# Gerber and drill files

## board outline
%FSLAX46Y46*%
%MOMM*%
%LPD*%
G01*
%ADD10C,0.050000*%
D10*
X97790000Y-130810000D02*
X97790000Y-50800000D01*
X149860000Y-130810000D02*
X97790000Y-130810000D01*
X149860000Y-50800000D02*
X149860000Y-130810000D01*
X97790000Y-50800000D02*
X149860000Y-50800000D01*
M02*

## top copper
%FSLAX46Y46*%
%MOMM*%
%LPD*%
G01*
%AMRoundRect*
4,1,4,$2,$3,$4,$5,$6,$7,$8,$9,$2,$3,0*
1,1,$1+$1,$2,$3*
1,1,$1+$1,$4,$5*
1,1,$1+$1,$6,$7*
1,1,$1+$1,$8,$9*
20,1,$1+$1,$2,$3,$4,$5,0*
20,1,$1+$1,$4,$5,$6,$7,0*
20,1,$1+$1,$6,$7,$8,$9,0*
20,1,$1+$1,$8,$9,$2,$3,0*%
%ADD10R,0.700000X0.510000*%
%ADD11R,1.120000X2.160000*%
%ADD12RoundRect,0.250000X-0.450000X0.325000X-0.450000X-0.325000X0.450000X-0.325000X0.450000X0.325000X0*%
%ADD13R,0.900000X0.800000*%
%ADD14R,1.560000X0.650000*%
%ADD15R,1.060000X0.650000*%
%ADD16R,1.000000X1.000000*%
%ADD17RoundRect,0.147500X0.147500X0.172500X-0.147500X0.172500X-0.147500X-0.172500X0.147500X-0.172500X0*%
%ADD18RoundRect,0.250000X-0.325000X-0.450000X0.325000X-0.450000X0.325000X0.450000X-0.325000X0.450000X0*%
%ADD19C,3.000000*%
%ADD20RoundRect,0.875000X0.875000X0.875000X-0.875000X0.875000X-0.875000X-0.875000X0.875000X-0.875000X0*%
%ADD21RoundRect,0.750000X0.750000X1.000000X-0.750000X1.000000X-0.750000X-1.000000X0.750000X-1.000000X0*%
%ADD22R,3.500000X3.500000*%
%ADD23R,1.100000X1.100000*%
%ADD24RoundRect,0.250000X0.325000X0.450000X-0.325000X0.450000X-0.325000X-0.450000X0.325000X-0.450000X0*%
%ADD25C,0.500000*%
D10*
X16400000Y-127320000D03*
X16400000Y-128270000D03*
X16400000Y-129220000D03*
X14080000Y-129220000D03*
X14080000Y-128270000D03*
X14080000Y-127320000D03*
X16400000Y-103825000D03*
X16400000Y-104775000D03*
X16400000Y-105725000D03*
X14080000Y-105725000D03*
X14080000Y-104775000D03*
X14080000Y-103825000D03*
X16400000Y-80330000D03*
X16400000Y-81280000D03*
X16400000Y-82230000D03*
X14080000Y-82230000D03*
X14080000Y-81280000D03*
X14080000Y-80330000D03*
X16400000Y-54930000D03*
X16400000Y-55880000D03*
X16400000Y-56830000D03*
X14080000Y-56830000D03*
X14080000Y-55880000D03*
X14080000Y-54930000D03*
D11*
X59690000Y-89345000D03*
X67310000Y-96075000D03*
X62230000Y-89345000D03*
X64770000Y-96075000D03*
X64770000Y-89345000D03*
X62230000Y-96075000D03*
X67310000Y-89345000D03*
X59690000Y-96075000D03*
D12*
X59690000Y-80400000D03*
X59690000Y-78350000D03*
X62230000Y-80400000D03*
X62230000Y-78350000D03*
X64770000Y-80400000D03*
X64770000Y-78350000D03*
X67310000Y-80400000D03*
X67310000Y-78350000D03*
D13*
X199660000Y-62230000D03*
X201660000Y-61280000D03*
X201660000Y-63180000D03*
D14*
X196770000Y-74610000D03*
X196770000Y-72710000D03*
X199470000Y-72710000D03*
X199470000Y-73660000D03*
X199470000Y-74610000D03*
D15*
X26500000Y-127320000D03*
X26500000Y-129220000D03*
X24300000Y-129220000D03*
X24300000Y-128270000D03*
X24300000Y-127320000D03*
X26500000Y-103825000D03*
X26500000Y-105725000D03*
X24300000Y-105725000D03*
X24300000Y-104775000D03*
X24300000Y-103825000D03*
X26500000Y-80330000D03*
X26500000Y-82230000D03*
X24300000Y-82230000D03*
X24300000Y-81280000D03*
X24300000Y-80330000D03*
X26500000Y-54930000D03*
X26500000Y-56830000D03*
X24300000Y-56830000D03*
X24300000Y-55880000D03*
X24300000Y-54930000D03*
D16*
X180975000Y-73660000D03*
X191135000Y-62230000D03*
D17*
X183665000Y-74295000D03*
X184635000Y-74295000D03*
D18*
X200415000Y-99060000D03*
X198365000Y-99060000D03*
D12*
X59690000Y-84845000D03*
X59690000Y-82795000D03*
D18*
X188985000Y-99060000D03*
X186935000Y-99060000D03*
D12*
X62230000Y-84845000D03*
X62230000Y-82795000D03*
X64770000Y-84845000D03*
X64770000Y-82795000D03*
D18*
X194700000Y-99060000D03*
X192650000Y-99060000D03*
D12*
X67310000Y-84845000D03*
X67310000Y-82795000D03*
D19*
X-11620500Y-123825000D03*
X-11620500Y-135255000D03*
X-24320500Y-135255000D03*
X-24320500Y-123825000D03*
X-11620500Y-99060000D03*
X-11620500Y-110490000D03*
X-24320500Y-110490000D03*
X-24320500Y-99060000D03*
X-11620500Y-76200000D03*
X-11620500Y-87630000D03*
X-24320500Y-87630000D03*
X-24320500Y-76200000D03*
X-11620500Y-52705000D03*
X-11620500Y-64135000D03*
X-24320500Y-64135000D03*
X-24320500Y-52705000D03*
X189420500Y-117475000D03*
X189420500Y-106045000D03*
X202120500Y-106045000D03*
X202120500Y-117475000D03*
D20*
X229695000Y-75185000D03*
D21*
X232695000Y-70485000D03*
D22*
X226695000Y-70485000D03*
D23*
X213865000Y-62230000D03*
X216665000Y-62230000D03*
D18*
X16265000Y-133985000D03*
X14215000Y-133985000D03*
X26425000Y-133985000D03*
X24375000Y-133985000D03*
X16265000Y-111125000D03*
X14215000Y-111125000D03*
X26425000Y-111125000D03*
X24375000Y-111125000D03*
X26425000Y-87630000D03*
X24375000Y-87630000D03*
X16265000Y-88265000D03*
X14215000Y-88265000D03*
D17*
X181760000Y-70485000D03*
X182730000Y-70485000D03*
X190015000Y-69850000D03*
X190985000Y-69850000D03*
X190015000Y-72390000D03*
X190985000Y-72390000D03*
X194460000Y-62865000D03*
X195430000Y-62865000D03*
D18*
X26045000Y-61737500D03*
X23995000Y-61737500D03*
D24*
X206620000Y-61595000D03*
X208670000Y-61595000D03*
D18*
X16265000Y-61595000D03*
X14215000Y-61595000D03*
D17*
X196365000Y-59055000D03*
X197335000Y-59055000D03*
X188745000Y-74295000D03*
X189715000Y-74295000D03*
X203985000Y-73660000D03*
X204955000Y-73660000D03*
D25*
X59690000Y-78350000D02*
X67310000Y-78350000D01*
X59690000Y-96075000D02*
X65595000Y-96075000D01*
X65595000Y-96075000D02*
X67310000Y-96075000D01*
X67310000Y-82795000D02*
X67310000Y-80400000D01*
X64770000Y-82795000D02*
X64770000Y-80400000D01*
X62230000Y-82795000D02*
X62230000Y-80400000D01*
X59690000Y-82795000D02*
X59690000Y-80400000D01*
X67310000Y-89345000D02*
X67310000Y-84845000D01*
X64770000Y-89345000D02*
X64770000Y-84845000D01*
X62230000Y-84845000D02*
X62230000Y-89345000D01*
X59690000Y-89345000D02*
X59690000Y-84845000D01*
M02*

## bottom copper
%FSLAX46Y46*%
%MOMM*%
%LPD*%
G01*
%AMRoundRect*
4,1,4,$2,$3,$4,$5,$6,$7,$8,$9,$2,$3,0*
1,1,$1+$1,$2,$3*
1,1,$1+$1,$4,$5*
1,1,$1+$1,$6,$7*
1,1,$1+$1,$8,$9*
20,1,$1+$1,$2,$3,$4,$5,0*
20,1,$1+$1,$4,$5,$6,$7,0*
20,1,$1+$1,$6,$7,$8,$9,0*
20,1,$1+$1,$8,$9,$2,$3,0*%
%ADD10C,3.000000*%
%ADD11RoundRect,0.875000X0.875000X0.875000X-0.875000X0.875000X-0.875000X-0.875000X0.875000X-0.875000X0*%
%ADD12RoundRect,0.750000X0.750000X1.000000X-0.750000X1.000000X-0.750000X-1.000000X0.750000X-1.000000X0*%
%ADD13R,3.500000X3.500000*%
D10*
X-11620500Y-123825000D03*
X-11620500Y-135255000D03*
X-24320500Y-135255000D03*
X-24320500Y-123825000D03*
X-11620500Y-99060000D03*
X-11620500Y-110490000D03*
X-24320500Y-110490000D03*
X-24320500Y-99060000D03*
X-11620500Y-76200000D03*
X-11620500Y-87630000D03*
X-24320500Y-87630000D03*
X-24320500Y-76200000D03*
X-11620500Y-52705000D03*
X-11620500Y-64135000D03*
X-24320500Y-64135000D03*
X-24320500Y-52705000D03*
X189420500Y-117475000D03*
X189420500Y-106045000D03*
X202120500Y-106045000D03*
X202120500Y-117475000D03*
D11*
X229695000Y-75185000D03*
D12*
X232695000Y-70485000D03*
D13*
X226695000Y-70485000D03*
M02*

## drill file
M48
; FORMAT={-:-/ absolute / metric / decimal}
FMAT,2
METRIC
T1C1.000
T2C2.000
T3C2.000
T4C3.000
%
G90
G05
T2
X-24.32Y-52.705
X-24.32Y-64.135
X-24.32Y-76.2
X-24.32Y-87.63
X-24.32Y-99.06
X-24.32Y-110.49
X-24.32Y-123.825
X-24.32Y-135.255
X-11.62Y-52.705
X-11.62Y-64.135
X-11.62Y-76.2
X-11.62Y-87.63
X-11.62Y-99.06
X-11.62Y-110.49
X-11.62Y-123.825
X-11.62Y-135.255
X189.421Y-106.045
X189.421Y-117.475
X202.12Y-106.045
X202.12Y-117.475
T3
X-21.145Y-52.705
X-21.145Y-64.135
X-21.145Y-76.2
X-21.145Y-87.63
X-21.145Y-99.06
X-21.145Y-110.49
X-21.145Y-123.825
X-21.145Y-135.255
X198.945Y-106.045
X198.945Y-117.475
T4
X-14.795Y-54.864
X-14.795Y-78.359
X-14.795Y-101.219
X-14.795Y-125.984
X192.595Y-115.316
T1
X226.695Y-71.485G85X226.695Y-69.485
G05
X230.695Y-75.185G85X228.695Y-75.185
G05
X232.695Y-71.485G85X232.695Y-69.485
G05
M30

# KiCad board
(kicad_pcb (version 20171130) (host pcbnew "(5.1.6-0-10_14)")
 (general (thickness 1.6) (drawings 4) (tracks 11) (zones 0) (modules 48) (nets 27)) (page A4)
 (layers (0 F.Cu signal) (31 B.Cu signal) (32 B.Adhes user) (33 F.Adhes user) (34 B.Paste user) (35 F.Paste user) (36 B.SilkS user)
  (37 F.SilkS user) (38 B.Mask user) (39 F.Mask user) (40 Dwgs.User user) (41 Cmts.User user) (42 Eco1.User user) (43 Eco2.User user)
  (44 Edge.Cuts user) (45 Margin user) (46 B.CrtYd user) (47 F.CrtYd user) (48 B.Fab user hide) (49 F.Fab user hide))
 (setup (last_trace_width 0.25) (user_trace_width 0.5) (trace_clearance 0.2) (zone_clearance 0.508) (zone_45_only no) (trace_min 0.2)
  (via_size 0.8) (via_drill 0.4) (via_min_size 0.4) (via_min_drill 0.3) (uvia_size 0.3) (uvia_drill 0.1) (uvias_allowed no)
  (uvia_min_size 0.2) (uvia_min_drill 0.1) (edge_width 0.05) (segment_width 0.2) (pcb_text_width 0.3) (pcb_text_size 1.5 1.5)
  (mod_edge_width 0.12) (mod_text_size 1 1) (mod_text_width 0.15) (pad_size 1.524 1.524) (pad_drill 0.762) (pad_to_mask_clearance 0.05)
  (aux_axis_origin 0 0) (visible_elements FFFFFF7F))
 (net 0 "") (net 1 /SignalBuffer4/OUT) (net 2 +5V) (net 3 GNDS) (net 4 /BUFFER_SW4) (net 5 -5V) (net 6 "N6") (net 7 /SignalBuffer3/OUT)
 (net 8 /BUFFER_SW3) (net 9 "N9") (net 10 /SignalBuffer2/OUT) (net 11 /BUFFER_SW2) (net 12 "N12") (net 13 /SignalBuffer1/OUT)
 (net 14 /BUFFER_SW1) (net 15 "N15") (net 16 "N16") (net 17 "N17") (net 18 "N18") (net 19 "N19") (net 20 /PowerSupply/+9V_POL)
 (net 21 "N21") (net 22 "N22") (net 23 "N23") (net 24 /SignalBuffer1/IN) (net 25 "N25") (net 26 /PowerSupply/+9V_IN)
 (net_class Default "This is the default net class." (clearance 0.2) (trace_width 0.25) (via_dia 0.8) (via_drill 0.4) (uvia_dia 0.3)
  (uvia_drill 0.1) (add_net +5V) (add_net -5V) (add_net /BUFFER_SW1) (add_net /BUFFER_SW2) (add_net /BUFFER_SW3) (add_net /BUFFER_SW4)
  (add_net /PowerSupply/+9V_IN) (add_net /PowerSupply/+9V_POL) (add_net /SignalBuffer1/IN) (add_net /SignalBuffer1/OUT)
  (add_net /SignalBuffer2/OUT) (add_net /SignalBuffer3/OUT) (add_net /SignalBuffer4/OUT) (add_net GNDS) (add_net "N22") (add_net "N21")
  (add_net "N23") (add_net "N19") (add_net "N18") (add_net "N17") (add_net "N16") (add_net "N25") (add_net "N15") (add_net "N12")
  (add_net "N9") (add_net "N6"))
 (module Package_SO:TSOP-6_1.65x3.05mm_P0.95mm (layer F.Cu) (at 15.24 128.27)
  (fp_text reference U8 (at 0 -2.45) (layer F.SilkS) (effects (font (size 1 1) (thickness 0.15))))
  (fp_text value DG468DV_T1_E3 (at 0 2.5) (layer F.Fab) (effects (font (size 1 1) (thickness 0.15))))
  (pad 6 smd rect (at 1.16 -0.95) (size 0.7 0.51) (layers F.Cu F.Paste F.Mask) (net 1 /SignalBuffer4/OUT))
  (pad 5 smd rect (at 1.16 0) (size 0.7 0.51) (layers F.Cu F.Paste F.Mask) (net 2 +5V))
  (pad 4 smd rect (at 1.16 0.95) (size 0.7 0.51) (layers F.Cu F.Paste F.Mask) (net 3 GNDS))
  (pad 3 smd rect (at -1.16 0.95) (size 0.7 0.51) (layers F.Cu F.Paste F.Mask) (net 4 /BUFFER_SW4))
  (pad 2 smd rect (at -1.16 0) (size 0.7 0.51) (layers F.Cu F.Paste F.Mask) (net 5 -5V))
  (pad 1 smd rect (at -1.16 -0.95) (size 0.7 0.51) (layers F.Cu F.Paste F.Mask) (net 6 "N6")))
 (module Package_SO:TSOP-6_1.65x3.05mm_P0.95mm (layer F.Cu) (at 15.24 104.775)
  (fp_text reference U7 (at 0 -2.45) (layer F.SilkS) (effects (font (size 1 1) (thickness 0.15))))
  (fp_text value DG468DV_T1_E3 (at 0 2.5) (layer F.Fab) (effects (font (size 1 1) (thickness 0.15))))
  (pad 6 smd rect (at 1.16 -0.95) (size 0.7 0.51) (layers F.Cu F.Paste F.Mask) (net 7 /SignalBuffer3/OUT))
  (pad 5 smd rect (at 1.16 0) (size 0.7 0.51) (layers F.Cu F.Paste F.Mask) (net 2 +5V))
  (pad 4 smd rect (at 1.16 0.95) (size 0.7 0.51) (layers F.Cu F.Paste F.Mask) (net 3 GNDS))
  (pad 3 smd rect (at -1.16 0.95) (size 0.7 0.51) (layers F.Cu F.Paste F.Mask) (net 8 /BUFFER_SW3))
  (pad 2 smd rect (at -1.16 0) (size 0.7 0.51) (layers F.Cu F.Paste F.Mask) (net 5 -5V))
  (pad 1 smd rect (at -1.16 -0.95) (size 0.7 0.51) (layers F.Cu F.Paste F.Mask) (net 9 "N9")))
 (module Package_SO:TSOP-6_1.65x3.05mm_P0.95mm (layer F.Cu) (at 15.24 81.28)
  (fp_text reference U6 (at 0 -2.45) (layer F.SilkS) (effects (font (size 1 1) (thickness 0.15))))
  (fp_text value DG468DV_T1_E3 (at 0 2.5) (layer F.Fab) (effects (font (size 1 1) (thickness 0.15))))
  (pad 6 smd rect (at 1.16 -0.95) (size 0.7 0.51) (layers F.Cu F.Paste F.Mask) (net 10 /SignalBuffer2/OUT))
  (pad 5 smd rect (at 1.16 0) (size 0.7 0.51) (layers F.Cu F.Paste F.Mask) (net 2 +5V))
  (pad 4 smd rect (at 1.16 0.95) (size 0.7 0.51) (layers F.Cu F.Paste F.Mask) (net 3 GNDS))
  (pad 3 smd rect (at -1.16 0.95) (size 0.7 0.51) (layers F.Cu F.Paste F.Mask) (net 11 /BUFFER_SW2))
  (pad 2 smd rect (at -1.16 0) (size 0.7 0.51) (layers F.Cu F.Paste F.Mask) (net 5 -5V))
  (pad 1 smd rect (at -1.16 -0.95) (size 0.7 0.51) (layers F.Cu F.Paste F.Mask) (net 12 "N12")))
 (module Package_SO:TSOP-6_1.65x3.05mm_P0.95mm (layer F.Cu) (at 15.24 55.88)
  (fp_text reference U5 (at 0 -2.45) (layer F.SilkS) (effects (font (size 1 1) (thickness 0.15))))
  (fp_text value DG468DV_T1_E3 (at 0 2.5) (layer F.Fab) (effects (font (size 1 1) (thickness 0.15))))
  (pad 6 smd rect (at 1.16 -0.95) (size 0.7 0.51) (layers F.Cu F.Paste F.Mask) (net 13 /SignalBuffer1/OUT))
  (pad 5 smd rect (at 1.16 0) (size 0.7 0.51) (layers F.Cu F.Paste F.Mask) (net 2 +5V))
  (pad 4 smd rect (at 1.16 0.95) (size 0.7 0.51) (layers F.Cu F.Paste F.Mask) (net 3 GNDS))
  (pad 3 smd rect (at -1.16 0.95) (size 0.7 0.51) (layers F.Cu F.Paste F.Mask) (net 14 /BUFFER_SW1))
  (pad 2 smd rect (at -1.16 0) (size 0.7 0.51) (layers F.Cu F.Paste F.Mask) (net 5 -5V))
  (pad 1 smd rect (at -1.16 -0.95) (size 0.7 0.51) (layers F.Cu F.Paste F.Mask) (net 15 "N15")))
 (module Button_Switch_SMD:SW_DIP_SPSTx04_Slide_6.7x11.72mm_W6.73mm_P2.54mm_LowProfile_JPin (layer F.Cu) (at 63.5 92.71 90)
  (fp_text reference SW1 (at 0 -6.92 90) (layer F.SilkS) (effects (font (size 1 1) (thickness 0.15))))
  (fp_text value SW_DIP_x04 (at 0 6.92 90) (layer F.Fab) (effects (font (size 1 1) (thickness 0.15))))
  (pad 8 smd rect (at 3.365 -3.81 90) (size 2.16 1.12) (layers F.Cu F.Paste F.Mask) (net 14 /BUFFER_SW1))
  (pad 4 smd rect (at -3.365 3.81 90) (size 2.16 1.12) (layers F.Cu F.Paste F.Mask) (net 2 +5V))
  (pad 7 smd rect (at 3.365 -1.27 90) (size 2.16 1.12) (layers F.Cu F.Paste F.Mask) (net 11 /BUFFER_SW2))
  (pad 3 smd rect (at -3.365 1.27 90) (size 2.16 1.12) (layers F.Cu F.Paste F.Mask) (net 2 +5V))
  (pad 6 smd rect (at 3.365 1.27 90) (size 2.16 1.12) (layers F.Cu F.Paste F.Mask) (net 8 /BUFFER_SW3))
  (pad 2 smd rect (at -3.365 -1.27 90) (size 2.16 1.12) (layers F.Cu F.Paste F.Mask) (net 2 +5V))
  (pad 5 smd rect (at 3.365 3.81 90) (size 2.16 1.12) (layers F.Cu F.Paste F.Mask) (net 4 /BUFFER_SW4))
  (pad 1 smd rect (at -3.365 -3.81 90) (size 2.16 1.12) (layers F.Cu F.Paste F.Mask) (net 2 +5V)))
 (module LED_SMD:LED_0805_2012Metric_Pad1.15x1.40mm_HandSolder (layer F.Cu) (at 59.69 79.375 270)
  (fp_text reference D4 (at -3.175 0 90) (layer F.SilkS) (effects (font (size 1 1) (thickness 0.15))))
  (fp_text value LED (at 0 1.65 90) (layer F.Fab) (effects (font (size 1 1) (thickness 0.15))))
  (pad 2 smd roundrect (at 1.025 0 270) (size 1.15 1.4) (layers F.Cu F.Paste F.Mask) (roundrect_rratio 0.217391) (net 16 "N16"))
  (pad 1 smd roundrect (at -1.025 0 270) (size 1.15 1.4) (layers F.Cu F.Paste F.Mask) (roundrect_rratio 0.217391) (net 3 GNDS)))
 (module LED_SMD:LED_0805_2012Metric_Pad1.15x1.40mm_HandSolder (layer F.Cu) (at 62.23 79.375 270)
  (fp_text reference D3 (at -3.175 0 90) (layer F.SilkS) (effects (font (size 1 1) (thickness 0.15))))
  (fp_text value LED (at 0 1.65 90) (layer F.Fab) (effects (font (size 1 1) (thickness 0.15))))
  (pad 2 smd roundrect (at 1.025 0 270) (size 1.15 1.4) (layers F.Cu F.Paste F.Mask) (roundrect_rratio 0.217391) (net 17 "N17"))
  (pad 1 smd roundrect (at -1.025 0 270) (size 1.15 1.4) (layers F.Cu F.Paste F.Mask) (roundrect_rratio 0.217391) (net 3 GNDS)))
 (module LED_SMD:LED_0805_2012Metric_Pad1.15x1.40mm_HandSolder (layer F.Cu) (at 64.77 79.375 270)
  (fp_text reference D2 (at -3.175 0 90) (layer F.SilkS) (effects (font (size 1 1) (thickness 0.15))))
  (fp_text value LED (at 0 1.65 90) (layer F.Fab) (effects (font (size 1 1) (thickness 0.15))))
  (pad 2 smd roundrect (at 1.025 0 270) (size 1.15 1.4) (layers F.Cu F.Paste F.Mask) (roundrect_rratio 0.217391) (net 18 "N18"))
  (pad 1 smd roundrect (at -1.025 0 270) (size 1.15 1.4) (layers F.Cu F.Paste F.Mask) (roundrect_rratio 0.217391) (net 3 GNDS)))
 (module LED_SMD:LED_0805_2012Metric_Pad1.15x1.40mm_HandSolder (layer F.Cu) (at 67.31 79.375 270)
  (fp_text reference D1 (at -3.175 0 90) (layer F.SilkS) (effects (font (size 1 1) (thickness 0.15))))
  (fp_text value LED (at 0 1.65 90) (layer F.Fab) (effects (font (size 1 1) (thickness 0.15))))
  (pad 2 smd roundrect (at 1.025 0 270) (size 1.15 1.4) (layers F.Cu F.Paste F.Mask) (roundrect_rratio 0.217391) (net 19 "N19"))
  (pad 1 smd roundrect (at -1.025 0 270) (size 1.15 1.4) (layers F.Cu F.Paste F.Mask) (roundrect_rratio 0.217391) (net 3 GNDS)))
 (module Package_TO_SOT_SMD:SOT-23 (layer F.Cu) (at 200.66 62.23 180)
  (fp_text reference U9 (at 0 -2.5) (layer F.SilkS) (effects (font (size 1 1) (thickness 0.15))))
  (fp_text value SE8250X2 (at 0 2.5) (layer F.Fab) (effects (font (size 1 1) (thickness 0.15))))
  (pad 3 smd rect (at 1 0 180) (size 0.9 0.8) (layers F.Cu F.Paste F.Mask) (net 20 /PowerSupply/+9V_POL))
  (pad 2 smd rect (at -1 0.95 180) (size 0.9 0.8) (layers F.Cu F.Paste F.Mask) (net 2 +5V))
  (pad 1 smd rect (at -1 -0.95 180) (size 0.9 0.8) (layers F.Cu F.Paste F.Mask) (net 3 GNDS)))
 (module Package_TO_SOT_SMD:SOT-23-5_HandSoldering (layer F.Cu) (at 198.12 73.66 180)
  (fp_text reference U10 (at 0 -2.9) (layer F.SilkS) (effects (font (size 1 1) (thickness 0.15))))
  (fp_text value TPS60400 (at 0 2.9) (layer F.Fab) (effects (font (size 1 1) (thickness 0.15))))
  (pad 5 smd rect (at 1.35 -0.95 180) (size 1.56 0.65) (layers F.Cu F.Paste F.Mask) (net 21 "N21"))
  (pad 4 smd rect (at 1.35 0.95 180) (size 1.56 0.65) (layers F.Cu F.Paste F.Mask) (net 3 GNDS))
  (pad 3 smd rect (at -1.35 0.95 180) (size 1.56 0.65) (layers F.Cu F.Paste F.Mask) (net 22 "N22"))
  (pad 2 smd rect (at -1.35 0 180) (size 1.56 0.65) (layers F.Cu F.Paste F.Mask) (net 2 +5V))
  (pad 1 smd rect (at -1.35 -0.95 180) (size 1.56 0.65) (layers F.Cu F.Paste F.Mask) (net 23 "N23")))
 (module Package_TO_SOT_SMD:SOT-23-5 (layer F.Cu) (at 25.4 128.27)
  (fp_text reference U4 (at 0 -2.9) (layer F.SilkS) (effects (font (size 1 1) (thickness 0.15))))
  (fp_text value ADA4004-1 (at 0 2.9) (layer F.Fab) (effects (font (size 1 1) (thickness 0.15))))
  (pad 5 smd rect (at 1.1 -0.95) (size 1.06 0.65) (layers F.Cu F.Paste F.Mask) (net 2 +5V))
  (pad 4 smd rect (at 1.1 0.95) (size 1.06 0.65) (layers F.Cu F.Paste F.Mask) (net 6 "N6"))
  (pad 3 smd rect (at -1.1 0.95) (size 1.06 0.65) (layers F.Cu F.Paste F.Mask) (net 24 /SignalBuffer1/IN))
  (pad 2 smd rect (at -1.1 0) (size 1.06 0.65) (layers F.Cu F.Paste F.Mask) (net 5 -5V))
  (pad 1 smd rect (at -1.1 -0.95) (size 1.06 0.65) (layers F.Cu F.Paste F.Mask) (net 6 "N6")))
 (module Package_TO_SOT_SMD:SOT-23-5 (layer F.Cu) (at 25.4 104.775)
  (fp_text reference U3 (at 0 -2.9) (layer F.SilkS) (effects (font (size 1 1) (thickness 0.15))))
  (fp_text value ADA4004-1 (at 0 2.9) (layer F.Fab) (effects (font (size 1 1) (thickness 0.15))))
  (pad 5 smd rect (at 1.1 -0.95) (size 1.06 0.65) (layers F.Cu F.Paste F.Mask) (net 2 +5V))
  (pad 4 smd rect (at 1.1 0.95) (size 1.06 0.65) (layers F.Cu F.Paste F.Mask) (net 9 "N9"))
  (pad 3 smd rect (at -1.1 0.95) (size 1.06 0.65) (layers F.Cu F.Paste F.Mask) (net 24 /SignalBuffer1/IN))
  (pad 2 smd rect (at -1.1 0) (size 1.06 0.65) (layers F.Cu F.Paste F.Mask) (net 5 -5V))
  (pad 1 smd rect (at -1.1 -0.95) (size 1.06 0.65) (layers F.Cu F.Paste F.Mask) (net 9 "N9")))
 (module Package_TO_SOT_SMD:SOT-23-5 (layer F.Cu) (at 25.4 81.28)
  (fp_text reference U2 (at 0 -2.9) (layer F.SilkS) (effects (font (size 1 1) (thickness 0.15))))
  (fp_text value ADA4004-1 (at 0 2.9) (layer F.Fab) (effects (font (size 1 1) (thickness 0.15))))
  (pad 5 smd rect (at 1.1 -0.95) (size 1.06 0.65) (layers F.Cu F.Paste F.Mask) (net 2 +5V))
  (pad 4 smd rect (at 1.1 0.95) (size 1.06 0.65) (layers F.Cu F.Paste F.Mask) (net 12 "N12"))
  (pad 3 smd rect (at -1.1 0.95) (size 1.06 0.65) (layers F.Cu F.Paste F.Mask) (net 24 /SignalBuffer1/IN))
  (pad 2 smd rect (at -1.1 0) (size 1.06 0.65) (layers F.Cu F.Paste F.Mask) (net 5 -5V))
  (pad 1 smd rect (at -1.1 -0.95) (size 1.06 0.65) (layers F.Cu F.Paste F.Mask) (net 12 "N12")))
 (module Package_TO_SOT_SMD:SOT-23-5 (layer F.Cu) (at 25.4 55.88)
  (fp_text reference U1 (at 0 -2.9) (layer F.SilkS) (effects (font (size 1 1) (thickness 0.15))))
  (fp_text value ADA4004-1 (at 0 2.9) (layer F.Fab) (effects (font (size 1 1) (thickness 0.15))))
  (pad 5 smd rect (at 1.1 -0.95) (size 1.06 0.65) (layers F.Cu F.Paste F.Mask) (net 2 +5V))
  (pad 4 smd rect (at 1.1 0.95) (size 1.06 0.65) (layers F.Cu F.Paste F.Mask) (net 15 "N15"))
  (pad 3 smd rect (at -1.1 0.95) (size 1.06 0.65) (layers F.Cu F.Paste F.Mask) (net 24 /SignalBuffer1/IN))
  (pad 2 smd rect (at -1.1 0) (size 1.06 0.65) (layers F.Cu F.Paste F.Mask) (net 5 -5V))
  (pad 1 smd rect (at -1.1 -0.95) (size 1.06 0.65) (layers F.Cu F.Paste F.Mask) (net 15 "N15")))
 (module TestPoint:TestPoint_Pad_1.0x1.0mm (layer F.Cu) (at 180.975 73.66 180)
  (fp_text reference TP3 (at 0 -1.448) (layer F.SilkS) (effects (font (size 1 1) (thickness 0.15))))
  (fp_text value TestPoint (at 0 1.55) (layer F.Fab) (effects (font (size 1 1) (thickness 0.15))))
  (pad 1 smd rect (at 0 0 180) (size 1 1) (layers F.Cu F.Mask) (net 5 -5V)))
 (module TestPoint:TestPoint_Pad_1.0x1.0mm (layer F.Cu) (at 191.135 62.23 180)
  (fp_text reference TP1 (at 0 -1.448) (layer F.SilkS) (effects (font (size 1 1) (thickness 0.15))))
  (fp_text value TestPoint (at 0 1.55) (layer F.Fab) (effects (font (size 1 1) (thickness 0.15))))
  (pad 1 smd rect (at 0 0 180) (size 1 1) (layers F.Cu F.Mask) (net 2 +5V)))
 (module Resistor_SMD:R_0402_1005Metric (layer F.Cu) (at 184.15 74.295 180)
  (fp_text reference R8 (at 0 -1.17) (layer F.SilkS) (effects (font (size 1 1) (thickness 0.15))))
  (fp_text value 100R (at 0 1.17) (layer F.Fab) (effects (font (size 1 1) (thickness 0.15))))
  (pad 2 smd roundrect (at 0.485 0 180) (size 0.59 0.64) (layers F.Cu F.Paste F.Mask) (roundrect_rratio 0.25) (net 5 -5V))
  (pad 1 smd roundrect (at -0.485 0 180) (size 0.59 0.64) (layers F.Cu F.Paste F.Mask) (roundrect_rratio 0.25) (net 23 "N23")))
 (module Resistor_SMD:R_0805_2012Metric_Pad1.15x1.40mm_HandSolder (layer F.Cu) (at 199.39 99.06)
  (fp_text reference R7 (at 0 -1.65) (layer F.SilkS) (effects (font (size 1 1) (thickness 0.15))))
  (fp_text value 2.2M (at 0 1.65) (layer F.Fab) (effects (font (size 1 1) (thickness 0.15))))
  (pad 2 smd roundrect (at 1.025 0) (size 1.15 1.4) (layers F.Cu F.Paste F.Mask) (roundrect_rratio 0.217391) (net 3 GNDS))
  (pad 1 smd roundrect (at -1.025 0) (size 1.15 1.4) (layers F.Cu F.Paste F.Mask) (roundrect_rratio 0.217391) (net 24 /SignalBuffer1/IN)))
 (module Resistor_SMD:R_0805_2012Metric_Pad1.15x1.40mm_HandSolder (layer F.Cu) (at 59.69 83.82 270)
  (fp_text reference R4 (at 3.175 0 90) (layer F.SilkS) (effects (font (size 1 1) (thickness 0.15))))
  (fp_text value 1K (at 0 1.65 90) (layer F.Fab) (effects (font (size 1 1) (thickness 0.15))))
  (pad 2 smd roundrect (at 1.025 0 270) (size 1.15 1.4) (layers F.Cu F.Paste F.Mask) (roundrect_rratio 0.217391) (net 14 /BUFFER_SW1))
  (pad 1 smd roundrect (at -1.025 0 270) (size 1.15 1.4) (layers F.Cu F.Paste F.Mask) (roundrect_rratio 0.217391) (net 16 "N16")))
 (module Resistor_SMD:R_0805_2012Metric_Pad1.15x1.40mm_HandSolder (layer F.Cu) (at 187.96 99.06)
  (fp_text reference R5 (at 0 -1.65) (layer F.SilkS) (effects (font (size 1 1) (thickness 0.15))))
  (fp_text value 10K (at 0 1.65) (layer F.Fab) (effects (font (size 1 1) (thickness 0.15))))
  (pad 2 smd roundrect (at 1.025 0) (size 1.15 1.4) (layers F.Cu F.Paste F.Mask) (roundrect_rratio 0.217391) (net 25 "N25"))
  (pad 1 smd roundrect (at -1.025 0) (size 1.15 1.4) (layers F.Cu F.Paste F.Mask) (roundrect_rratio 0.217391) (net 24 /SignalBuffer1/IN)))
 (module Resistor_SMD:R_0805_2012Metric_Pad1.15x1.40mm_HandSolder (layer F.Cu) (at 62.23 83.82 270)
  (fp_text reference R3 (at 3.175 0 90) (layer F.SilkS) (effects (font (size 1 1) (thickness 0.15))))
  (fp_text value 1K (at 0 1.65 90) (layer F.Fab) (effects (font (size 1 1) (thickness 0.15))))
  (pad 2 smd roundrect (at 1.025 0 270) (size 1.15 1.4) (layers F.Cu F.Paste F.Mask) (roundrect_rratio 0.217391) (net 11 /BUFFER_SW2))
  (pad 1 smd roundrect (at -1.025 0 270) (size 1.15 1.4) (layers F.Cu F.Paste F.Mask) (roundrect_rratio 0.217391) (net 17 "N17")))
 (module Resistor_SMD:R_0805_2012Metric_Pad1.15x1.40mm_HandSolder (layer F.Cu) (at 64.77 83.82 270)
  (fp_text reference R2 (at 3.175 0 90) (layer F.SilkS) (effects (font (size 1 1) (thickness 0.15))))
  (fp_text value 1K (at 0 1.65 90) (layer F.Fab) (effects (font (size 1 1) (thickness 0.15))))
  (pad 2 smd roundrect (at 1.025 0 270) (size 1.15 1.4) (layers F.Cu F.Paste F.Mask) (roundrect_rratio 0.217391) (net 8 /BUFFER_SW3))
  (pad 1 smd roundrect (at -1.025 0 270) (size 1.15 1.4) (layers F.Cu F.Paste F.Mask) (roundrect_rratio 0.217391) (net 18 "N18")))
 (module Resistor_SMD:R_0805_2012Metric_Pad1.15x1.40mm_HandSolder (layer F.Cu) (at 193.675 99.06)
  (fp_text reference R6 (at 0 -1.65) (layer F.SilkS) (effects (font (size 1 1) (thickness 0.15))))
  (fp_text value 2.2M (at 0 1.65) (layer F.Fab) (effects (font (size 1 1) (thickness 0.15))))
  (pad 2 smd roundrect (at 1.025 0) (size 1.15 1.4) (layers F.Cu F.Paste F.Mask) (roundrect_rratio 0.217391) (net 3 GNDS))
  (pad 1 smd roundrect (at -1.025 0) (size 1.15 1.4) (layers F.Cu F.Paste F.Mask) (roundrect_rratio 0.217391) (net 25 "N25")))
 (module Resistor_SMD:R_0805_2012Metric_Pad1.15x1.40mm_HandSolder (layer F.Cu) (at 67.31 83.82 270)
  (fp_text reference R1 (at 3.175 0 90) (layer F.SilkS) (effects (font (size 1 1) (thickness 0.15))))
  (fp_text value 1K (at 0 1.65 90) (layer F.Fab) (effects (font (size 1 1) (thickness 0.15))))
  (pad 2 smd roundrect (at 1.025 0 270) (size 1.15 1.4) (layers F.Cu F.Paste F.Mask) (roundrect_rratio 0.217391) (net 4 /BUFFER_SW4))
  (pad 1 smd roundrect (at -1.025 0 270) (size 1.15 1.4) (layers F.Cu F.Paste F.Mask) (roundrect_rratio 0.217391) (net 19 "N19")))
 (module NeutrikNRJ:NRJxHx (layer B.Cu) (at -17.78 129.54 180)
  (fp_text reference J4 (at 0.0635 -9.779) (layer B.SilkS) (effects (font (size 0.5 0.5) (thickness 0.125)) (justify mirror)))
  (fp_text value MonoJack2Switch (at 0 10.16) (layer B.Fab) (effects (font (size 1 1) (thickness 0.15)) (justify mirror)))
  (pad 1 thru_hole circle (at -6.1595 5.715 180) (size 3 3) (drill 2) (layers *.Cu *.Mask) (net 1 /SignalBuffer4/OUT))
  (pad 2 thru_hole circle (at -6.1595 -5.715 180) (size 3 3) (drill 2) (layers *.Cu *.Mask) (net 3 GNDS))
  (pad 3 thru_hole circle (at 6.5405 -5.715 180) (size 3 3) (drill 2) (layers *.Cu *.Mask) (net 3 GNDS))
  (pad 4 thru_hole circle (at 6.5405 5.715 180) (size 3 3) (drill 2) (layers *.Cu *.Mask) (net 3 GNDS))
  (pad "" np_thru_hole circle (at -2.9845 3.556 180) (size 3 3) (drill 3) (layers *.Cu *.Mask))
  (pad "" np_thru_hole circle (at 3.3655 5.715 180) (size 2 2) (drill 2) (layers *.Cu *.Mask))
  (pad "" np_thru_hole circle (at 3.3655 -5.715 180) (size 2 2) (drill 2) (layers *.Cu *.Mask)))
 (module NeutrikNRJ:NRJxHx (layer B.Cu) (at -17.78 104.775 180)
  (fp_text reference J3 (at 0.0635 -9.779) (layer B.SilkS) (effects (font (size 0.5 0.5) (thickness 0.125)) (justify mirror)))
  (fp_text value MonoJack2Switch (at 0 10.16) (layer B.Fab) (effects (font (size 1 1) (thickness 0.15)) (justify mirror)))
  (pad 1 thru_hole circle (at -6.1595 5.715 180) (size 3 3) (drill 2) (layers *.Cu *.Mask) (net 7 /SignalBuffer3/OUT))
  (pad 2 thru_hole circle (at -6.1595 -5.715 180) (size 3 3) (drill 2) (layers *.Cu *.Mask) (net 3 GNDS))
  (pad 3 thru_hole circle (at 6.5405 -5.715 180) (size 3 3) (drill 2) (layers *.Cu *.Mask) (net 3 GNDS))
  (pad 4 thru_hole circle (at 6.5405 5.715 180) (size 3 3) (drill 2) (layers *.Cu *.Mask) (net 3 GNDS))
  (pad "" np_thru_hole circle (at -2.9845 3.556 180) (size 3 3) (drill 3) (layers *.Cu *.Mask))
  (pad "" np_thru_hole circle (at 3.3655 5.715 180) (size 2 2) (drill 2) (layers *.Cu *.Mask))
  (pad "" np_thru_hole circle (at 3.3655 -5.715 180) (size 2 2) (drill 2) (layers *.Cu *.Mask)))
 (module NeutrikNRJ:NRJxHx (layer B.Cu) (at -17.78 81.915 180)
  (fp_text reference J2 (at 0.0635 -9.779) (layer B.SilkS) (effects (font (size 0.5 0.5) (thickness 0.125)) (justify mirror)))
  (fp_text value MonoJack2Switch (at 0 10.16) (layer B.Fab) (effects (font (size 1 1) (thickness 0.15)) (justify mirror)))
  (pad 1 thru_hole circle (at -6.1595 5.715 180) (size 3 3) (drill 2) (layers *.Cu *.Mask) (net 10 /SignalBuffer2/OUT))
  (pad 2 thru_hole circle (at -6.1595 -5.715 180) (size 3 3) (drill 2) (layers *.Cu *.Mask) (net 3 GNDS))
  (pad 3 thru_hole circle (at 6.5405 -5.715 180) (size 3 3) (drill 2) (layers *.Cu *.Mask) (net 3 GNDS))
  (pad 4 thru_hole circle (at 6.5405 5.715 180) (size 3 3) (drill 2) (layers *.Cu *.Mask) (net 3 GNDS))
  (pad "" np_thru_hole circle (at -2.9845 3.556 180) (size 3 3) (drill 3) (layers *.Cu *.Mask))
  (pad "" np_thru_hole circle (at 3.3655 5.715 180) (size 2 2) (drill 2) (layers *.Cu *.Mask))
  (pad "" np_thru_hole circle (at 3.3655 -5.715 180) (size 2 2) (drill 2) (layers *.Cu *.Mask)))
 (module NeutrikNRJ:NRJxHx (layer B.Cu) (at -17.78 58.42 180)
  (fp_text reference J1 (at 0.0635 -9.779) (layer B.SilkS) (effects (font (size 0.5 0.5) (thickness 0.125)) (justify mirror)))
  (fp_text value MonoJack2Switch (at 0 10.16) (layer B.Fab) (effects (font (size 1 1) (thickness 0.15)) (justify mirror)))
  (pad 1 thru_hole circle (at -6.1595 5.715 180) (size 3 3) (drill 2) (layers *.Cu *.Mask) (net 13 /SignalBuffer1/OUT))
  (pad 2 thru_hole circle (at -6.1595 -5.715 180) (size 3 3) (drill 2) (layers *.Cu *.Mask) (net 3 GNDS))
  (pad 3 thru_hole circle (at 6.5405 -5.715 180) (size 3 3) (drill 2) (layers *.Cu *.Mask) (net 3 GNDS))
  (pad 4 thru_hole circle (at 6.5405 5.715 180) (size 3 3) (drill 2) (layers *.Cu *.Mask) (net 3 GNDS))
  (pad "" np_thru_hole circle (at -2.9845 3.556 180) (size 3 3) (drill 3) (layers *.Cu *.Mask))
  (pad "" np_thru_hole circle (at 3.3655 5.715 180) (size 2 2) (drill 2) (layers *.Cu *.Mask))
  (pad "" np_thru_hole circle (at 3.3655 -5.715 180) (size 2 2) (drill 2) (layers *.Cu *.Mask)))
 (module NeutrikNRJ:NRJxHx (layer B.Cu) (at 195.58 111.76)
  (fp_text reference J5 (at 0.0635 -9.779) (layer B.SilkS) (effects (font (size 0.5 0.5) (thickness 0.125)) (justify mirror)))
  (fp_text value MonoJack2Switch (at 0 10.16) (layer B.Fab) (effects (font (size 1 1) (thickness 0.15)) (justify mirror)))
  (pad 1 thru_hole circle (at -6.1595 5.715) (size 3 3) (drill 2) (layers *.Cu *.Mask) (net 25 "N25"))
  (pad 2 thru_hole circle (at -6.1595 -5.715) (size 3 3) (drill 2) (layers *.Cu *.Mask) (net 3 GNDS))
  (pad 3 thru_hole circle (at 6.5405 -5.715) (size 3 3) (drill 2) (layers *.Cu *.Mask) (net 3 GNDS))
  (pad 4 thru_hole circle (at 6.5405 5.715) (size 3 3) (drill 2) (layers *.Cu *.Mask) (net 3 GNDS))
  (pad "" np_thru_hole circle (at -2.9845 3.556) (size 3 3) (drill 3) (layers *.Cu *.Mask))
  (pad "" np_thru_hole circle (at 3.3655 5.715) (size 2 2) (drill 2) (layers *.Cu *.Mask))
  (pad "" np_thru_hole circle (at 3.3655 -5.715) (size 2 2) (drill 2) (layers *.Cu *.Mask)))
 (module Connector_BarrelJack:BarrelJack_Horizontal (layer B.Cu) (at 226.695 70.485 180)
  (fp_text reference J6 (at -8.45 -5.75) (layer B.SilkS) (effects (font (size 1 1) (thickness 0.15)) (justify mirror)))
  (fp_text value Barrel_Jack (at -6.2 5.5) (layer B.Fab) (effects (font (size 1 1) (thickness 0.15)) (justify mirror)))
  (pad 3 thru_hole roundrect (at -3 -4.7 180) (size 3.5 3.5) (drill oval 3 1) (layers *.Cu *.Mask) (roundrect_rratio 0.25))
  (pad 2 thru_hole roundrect (at -6 0 180) (size 3 3.5) (drill oval 1 3) (layers *.Cu *.Mask) (roundrect_rratio 0.25)
   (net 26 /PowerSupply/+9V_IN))
  (pad 1 thru_hole rect (at 0 0 180) (size 3.5 3.5) (drill oval 1 3) (layers *.Cu *.Mask) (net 3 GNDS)))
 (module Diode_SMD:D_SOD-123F (layer F.Cu) (at 215.265 62.23 180)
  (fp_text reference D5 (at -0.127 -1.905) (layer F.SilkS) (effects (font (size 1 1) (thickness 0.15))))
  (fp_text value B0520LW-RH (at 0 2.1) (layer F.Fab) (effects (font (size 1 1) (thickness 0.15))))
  (pad 2 smd rect (at 1.4 0 180) (size 1.1 1.1) (layers F.Cu F.Paste F.Mask) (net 26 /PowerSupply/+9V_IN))
  (pad 1 smd rect (at -1.4 0 180) (size 1.1 1.1) (layers F.Cu F.Paste F.Mask) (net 20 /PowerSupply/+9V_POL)))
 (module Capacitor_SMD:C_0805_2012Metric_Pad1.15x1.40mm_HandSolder (layer F.Cu) (at 15.24 133.985)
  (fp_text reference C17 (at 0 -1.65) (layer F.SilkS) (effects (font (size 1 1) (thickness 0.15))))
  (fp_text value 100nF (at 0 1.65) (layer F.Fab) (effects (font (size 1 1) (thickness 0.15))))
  (pad 2 smd roundrect (at 1.025 0) (size 1.15 1.4) (layers F.Cu F.Paste F.Mask) (roundrect_rratio 0.217391) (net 3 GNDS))
  (pad 1 smd roundrect (at -1.025 0) (size 1.15 1.4) (layers F.Cu F.Paste F.Mask) (roundrect_rratio 0.217391) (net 2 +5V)))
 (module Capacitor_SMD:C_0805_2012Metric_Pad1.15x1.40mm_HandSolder (layer F.Cu) (at 25.4 133.985)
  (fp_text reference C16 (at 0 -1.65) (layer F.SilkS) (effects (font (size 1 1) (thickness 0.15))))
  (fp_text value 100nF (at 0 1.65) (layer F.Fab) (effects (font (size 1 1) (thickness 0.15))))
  (pad 2 smd roundrect (at 1.025 0) (size 1.15 1.4) (layers F.Cu F.Paste F.Mask) (roundrect_rratio 0.217391) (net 3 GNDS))
  (pad 1 smd roundrect (at -1.025 0) (size 1.15 1.4) (layers F.Cu F.Paste F.Mask) (roundrect_rratio 0.217391) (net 2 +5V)))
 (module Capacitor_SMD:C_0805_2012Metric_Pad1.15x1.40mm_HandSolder (layer F.Cu) (at 15.24 111.125)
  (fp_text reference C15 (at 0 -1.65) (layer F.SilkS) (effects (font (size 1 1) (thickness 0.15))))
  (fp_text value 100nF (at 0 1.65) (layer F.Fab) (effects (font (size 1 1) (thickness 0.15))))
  (pad 2 smd roundrect (at 1.025 0) (size 1.15 1.4) (layers F.Cu F.Paste F.Mask) (roundrect_rratio 0.217391) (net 3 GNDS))
  (pad 1 smd roundrect (at -1.025 0) (size 1.15 1.4) (layers F.Cu F.Paste F.Mask) (roundrect_rratio 0.217391) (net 2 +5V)))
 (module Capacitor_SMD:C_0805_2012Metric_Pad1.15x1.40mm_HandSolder (layer F.Cu) (at 25.4 111.125)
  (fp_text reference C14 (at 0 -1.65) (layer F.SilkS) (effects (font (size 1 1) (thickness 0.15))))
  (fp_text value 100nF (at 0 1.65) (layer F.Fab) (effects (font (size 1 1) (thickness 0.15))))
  (pad 2 smd roundrect (at 1.025 0) (size 1.15 1.4) (layers F.Cu F.Paste F.Mask) (roundrect_rratio 0.217391) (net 3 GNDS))
  (pad 1 smd roundrect (at -1.025 0) (size 1.15 1.4) (layers F.Cu F.Paste F.Mask) (roundrect_rratio 0.217391) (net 2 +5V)))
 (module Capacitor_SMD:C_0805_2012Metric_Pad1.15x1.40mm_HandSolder (layer F.Cu) (at 25.4 87.63)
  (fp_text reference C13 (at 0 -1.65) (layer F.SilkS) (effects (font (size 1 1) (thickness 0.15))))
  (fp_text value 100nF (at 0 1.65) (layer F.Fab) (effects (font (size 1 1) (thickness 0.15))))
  (pad 2 smd roundrect (at 1.025 0) (size 1.15 1.4) (layers F.Cu F.Paste F.Mask) (roundrect_rratio 0.217391) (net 3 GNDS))
  (pad 1 smd roundrect (at -1.025 0) (size 1.15 1.4) (layers F.Cu F.Paste F.Mask) (roundrect_rratio 0.217391) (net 2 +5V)))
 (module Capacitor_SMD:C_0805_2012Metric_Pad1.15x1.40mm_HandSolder (layer F.Cu) (at 15.24 88.265)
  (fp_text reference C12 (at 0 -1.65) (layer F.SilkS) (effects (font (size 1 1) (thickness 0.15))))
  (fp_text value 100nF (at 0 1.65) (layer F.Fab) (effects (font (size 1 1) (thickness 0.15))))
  (pad 2 smd roundrect (at 1.025 0) (size 1.15 1.4) (layers F.Cu F.Paste F.Mask) (roundrect_rratio 0.217391) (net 3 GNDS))
  (pad 1 smd roundrect (at -1.025 0) (size 1.15 1.4) (layers F.Cu F.Paste F.Mask) (roundrect_rratio 0.217391) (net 2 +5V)))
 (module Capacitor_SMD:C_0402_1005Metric (layer F.Cu) (at 182.245 70.485 180)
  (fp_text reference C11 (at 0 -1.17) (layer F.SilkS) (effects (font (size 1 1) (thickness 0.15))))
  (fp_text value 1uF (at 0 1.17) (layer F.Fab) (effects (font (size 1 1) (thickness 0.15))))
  (pad 2 smd roundrect (at 0.485 0 180) (size 0.59 0.64) (layers F.Cu F.Paste F.Mask) (roundrect_rratio 0.25) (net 3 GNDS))
  (pad 1 smd roundrect (at -0.485 0 180) (size 0.59 0.64) (layers F.Cu F.Paste F.Mask) (roundrect_rratio 0.25) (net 5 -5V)))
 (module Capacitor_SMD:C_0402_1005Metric (layer F.Cu) (at 190.5 69.85 180)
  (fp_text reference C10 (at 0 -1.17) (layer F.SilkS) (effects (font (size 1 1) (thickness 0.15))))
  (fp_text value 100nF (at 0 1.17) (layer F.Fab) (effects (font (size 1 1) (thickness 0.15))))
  (pad 2 smd roundrect (at 0.485 0 180) (size 0.59 0.64) (layers F.Cu F.Paste F.Mask) (roundrect_rratio 0.25) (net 3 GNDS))
  (pad 1 smd roundrect (at -0.485 0 180) (size 0.59 0.64) (layers F.Cu F.Paste F.Mask) (roundrect_rratio 0.25) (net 2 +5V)))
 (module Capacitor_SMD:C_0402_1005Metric (layer F.Cu) (at 190.5 72.39 180)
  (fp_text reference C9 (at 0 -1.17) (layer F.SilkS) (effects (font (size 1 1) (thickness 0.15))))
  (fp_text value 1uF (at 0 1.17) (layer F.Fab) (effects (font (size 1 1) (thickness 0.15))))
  (pad 2 smd roundrect (at 0.485 0 180) (size 0.59 0.64) (layers F.Cu F.Paste F.Mask) (roundrect_rratio 0.25) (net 3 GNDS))
  (pad 1 smd roundrect (at -0.485 0 180) (size 0.59 0.64) (layers F.Cu F.Paste F.Mask) (roundrect_rratio 0.25) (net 23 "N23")))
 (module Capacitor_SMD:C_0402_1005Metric (layer F.Cu) (at 194.945 62.865 180)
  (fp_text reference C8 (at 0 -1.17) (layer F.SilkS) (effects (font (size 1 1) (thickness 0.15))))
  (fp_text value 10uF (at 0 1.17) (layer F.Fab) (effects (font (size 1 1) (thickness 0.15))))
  (pad 2 smd roundrect (at 0.485 0 180) (size 0.59 0.64) (layers F.Cu F.Paste F.Mask) (roundrect_rratio 0.25) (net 3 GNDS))
  (pad 1 smd roundrect (at -0.485 0 180) (size 0.59 0.64) (layers F.Cu F.Paste F.Mask) (roundrect_rratio 0.25) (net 2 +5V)))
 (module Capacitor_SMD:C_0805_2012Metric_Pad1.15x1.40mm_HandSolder (layer F.Cu) (at 25.02 61.7375)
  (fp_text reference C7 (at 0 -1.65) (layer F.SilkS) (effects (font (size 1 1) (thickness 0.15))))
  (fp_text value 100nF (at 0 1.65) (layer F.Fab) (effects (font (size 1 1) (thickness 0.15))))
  (pad 2 smd roundrect (at 1.025 0) (size 1.15 1.4) (layers F.Cu F.Paste F.Mask) (roundrect_rratio 0.217391) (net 3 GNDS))
  (pad 1 smd roundrect (at -1.025 0) (size 1.15 1.4) (layers F.Cu F.Paste F.Mask) (roundrect_rratio 0.217391) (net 2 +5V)))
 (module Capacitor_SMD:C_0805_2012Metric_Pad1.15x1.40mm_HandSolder (layer F.Cu) (at 207.645 61.595 180)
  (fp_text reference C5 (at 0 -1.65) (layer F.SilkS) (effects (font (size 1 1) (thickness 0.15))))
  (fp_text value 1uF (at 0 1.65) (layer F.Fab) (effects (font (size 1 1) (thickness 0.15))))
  (pad 2 smd roundrect (at 1.025 0 180) (size 1.15 1.4) (layers F.Cu F.Paste F.Mask) (roundrect_rratio 0.217391) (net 3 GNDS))
  (pad 1 smd roundrect (at -1.025 0 180) (size 1.15 1.4) (layers F.Cu F.Paste F.Mask) (roundrect_rratio 0.217391)
   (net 20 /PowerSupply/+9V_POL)))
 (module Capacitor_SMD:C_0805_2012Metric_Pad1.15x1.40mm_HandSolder (layer F.Cu) (at 15.24 61.595)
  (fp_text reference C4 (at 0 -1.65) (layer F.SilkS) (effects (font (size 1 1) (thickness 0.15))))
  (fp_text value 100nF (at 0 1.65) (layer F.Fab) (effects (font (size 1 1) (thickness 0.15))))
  (pad 2 smd roundrect (at 1.025 0) (size 1.15 1.4) (layers F.Cu F.Paste F.Mask) (roundrect_rratio 0.217391) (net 3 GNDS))
  (pad 1 smd roundrect (at -1.025 0) (size 1.15 1.4) (layers F.Cu F.Paste F.Mask) (roundrect_rratio 0.217391) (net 2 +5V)))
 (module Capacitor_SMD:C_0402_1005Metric (layer F.Cu) (at 196.85 59.055 180)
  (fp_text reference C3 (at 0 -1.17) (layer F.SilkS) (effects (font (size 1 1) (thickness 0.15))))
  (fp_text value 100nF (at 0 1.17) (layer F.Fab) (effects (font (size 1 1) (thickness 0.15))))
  (pad 2 smd roundrect (at 0.485 0 180) (size 0.59 0.64) (layers F.Cu F.Paste F.Mask) (roundrect_rratio 0.25) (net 3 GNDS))
  (pad 1 smd roundrect (at -0.485 0 180) (size 0.59 0.64) (layers F.Cu F.Paste F.Mask) (roundrect_rratio 0.25) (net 5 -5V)))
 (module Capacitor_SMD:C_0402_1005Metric (layer F.Cu) (at 189.23 74.295 180)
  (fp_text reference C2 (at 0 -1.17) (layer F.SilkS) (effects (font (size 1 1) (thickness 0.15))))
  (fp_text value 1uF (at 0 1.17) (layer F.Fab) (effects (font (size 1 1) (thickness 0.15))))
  (pad 2 smd roundrect (at 0.485 0 180) (size 0.59 0.64) (layers F.Cu F.Paste F.Mask) (roundrect_rratio 0.25) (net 21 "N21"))
  (pad 1 smd roundrect (at -0.485 0 180) (size 0.59 0.64) (layers F.Cu F.Paste F.Mask) (roundrect_rratio 0.25) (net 22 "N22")))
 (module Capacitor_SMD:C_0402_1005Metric (layer F.Cu) (at 204.47 73.66 180)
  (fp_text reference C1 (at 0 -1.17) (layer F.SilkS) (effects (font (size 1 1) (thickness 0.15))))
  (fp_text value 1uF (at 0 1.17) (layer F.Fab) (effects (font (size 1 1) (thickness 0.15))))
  (pad 2 smd roundrect (at 0.485 0 180) (size 0.59 0.64) (layers F.Cu F.Paste F.Mask) (roundrect_rratio 0.25) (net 3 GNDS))
  (pad 1 smd roundrect (at -0.485 0 180) (size 0.59 0.64) (layers F.Cu F.Paste F.Mask) (roundrect_rratio 0.25) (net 2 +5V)))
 (gr_line (start 97.79 130.81) (end 97.79 50.8) (layer Edge.Cuts) (width 0.05))
 (gr_line (start 149.86 130.81) (end 97.79 130.81) (layer Edge.Cuts) (width 0.05))
 (gr_line (start 149.86 50.8) (end 149.86 130.81) (layer Edge.Cuts) (width 0.05))
 (gr_line (start 97.79 50.8) (end 149.86 50.8) (layer Edge.Cuts) (width 0.05))
 (segment (start 59.69 78.35) (end 67.31 78.35) (width 0.5) (layer F.Cu) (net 3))
 (segment (start 59.69 96.075) (end 65.595 96.075) (width 0.5) (layer F.Cu) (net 2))
 (segment (start 65.595 96.075) (end 67.31 96.075) (width 0.5) (layer F.Cu) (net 2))
 (segment (start 67.31 82.795) (end 67.31 80.4) (width 0.5) (layer F.Cu) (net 19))
 (segment (start 64.77 82.795) (end 64.77 80.4) (width 0.5) (layer F.Cu) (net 18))
 (segment (start 62.23 82.795) (end 62.23 80.4) (width 0.5) (layer F.Cu) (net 17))
 (segment (start 59.69 82.795) (end 59.69 80.4) (width 0.5) (layer F.Cu) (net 16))
 (segment (start 67.31 89.345) (end 67.31 84.845) (width 0.5) (layer F.Cu) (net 4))
 (segment (start 64.77 89.345) (end 64.77 84.845) (width 0.5) (layer F.Cu) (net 8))
 (segment (start 62.23 84.845) (end 62.23 89.345) (width 0.5) (layer F.Cu) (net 11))
 (segment (start 59.69 89.345) (end 59.69 84.845) (width 0.5) (layer F.Cu) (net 14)))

